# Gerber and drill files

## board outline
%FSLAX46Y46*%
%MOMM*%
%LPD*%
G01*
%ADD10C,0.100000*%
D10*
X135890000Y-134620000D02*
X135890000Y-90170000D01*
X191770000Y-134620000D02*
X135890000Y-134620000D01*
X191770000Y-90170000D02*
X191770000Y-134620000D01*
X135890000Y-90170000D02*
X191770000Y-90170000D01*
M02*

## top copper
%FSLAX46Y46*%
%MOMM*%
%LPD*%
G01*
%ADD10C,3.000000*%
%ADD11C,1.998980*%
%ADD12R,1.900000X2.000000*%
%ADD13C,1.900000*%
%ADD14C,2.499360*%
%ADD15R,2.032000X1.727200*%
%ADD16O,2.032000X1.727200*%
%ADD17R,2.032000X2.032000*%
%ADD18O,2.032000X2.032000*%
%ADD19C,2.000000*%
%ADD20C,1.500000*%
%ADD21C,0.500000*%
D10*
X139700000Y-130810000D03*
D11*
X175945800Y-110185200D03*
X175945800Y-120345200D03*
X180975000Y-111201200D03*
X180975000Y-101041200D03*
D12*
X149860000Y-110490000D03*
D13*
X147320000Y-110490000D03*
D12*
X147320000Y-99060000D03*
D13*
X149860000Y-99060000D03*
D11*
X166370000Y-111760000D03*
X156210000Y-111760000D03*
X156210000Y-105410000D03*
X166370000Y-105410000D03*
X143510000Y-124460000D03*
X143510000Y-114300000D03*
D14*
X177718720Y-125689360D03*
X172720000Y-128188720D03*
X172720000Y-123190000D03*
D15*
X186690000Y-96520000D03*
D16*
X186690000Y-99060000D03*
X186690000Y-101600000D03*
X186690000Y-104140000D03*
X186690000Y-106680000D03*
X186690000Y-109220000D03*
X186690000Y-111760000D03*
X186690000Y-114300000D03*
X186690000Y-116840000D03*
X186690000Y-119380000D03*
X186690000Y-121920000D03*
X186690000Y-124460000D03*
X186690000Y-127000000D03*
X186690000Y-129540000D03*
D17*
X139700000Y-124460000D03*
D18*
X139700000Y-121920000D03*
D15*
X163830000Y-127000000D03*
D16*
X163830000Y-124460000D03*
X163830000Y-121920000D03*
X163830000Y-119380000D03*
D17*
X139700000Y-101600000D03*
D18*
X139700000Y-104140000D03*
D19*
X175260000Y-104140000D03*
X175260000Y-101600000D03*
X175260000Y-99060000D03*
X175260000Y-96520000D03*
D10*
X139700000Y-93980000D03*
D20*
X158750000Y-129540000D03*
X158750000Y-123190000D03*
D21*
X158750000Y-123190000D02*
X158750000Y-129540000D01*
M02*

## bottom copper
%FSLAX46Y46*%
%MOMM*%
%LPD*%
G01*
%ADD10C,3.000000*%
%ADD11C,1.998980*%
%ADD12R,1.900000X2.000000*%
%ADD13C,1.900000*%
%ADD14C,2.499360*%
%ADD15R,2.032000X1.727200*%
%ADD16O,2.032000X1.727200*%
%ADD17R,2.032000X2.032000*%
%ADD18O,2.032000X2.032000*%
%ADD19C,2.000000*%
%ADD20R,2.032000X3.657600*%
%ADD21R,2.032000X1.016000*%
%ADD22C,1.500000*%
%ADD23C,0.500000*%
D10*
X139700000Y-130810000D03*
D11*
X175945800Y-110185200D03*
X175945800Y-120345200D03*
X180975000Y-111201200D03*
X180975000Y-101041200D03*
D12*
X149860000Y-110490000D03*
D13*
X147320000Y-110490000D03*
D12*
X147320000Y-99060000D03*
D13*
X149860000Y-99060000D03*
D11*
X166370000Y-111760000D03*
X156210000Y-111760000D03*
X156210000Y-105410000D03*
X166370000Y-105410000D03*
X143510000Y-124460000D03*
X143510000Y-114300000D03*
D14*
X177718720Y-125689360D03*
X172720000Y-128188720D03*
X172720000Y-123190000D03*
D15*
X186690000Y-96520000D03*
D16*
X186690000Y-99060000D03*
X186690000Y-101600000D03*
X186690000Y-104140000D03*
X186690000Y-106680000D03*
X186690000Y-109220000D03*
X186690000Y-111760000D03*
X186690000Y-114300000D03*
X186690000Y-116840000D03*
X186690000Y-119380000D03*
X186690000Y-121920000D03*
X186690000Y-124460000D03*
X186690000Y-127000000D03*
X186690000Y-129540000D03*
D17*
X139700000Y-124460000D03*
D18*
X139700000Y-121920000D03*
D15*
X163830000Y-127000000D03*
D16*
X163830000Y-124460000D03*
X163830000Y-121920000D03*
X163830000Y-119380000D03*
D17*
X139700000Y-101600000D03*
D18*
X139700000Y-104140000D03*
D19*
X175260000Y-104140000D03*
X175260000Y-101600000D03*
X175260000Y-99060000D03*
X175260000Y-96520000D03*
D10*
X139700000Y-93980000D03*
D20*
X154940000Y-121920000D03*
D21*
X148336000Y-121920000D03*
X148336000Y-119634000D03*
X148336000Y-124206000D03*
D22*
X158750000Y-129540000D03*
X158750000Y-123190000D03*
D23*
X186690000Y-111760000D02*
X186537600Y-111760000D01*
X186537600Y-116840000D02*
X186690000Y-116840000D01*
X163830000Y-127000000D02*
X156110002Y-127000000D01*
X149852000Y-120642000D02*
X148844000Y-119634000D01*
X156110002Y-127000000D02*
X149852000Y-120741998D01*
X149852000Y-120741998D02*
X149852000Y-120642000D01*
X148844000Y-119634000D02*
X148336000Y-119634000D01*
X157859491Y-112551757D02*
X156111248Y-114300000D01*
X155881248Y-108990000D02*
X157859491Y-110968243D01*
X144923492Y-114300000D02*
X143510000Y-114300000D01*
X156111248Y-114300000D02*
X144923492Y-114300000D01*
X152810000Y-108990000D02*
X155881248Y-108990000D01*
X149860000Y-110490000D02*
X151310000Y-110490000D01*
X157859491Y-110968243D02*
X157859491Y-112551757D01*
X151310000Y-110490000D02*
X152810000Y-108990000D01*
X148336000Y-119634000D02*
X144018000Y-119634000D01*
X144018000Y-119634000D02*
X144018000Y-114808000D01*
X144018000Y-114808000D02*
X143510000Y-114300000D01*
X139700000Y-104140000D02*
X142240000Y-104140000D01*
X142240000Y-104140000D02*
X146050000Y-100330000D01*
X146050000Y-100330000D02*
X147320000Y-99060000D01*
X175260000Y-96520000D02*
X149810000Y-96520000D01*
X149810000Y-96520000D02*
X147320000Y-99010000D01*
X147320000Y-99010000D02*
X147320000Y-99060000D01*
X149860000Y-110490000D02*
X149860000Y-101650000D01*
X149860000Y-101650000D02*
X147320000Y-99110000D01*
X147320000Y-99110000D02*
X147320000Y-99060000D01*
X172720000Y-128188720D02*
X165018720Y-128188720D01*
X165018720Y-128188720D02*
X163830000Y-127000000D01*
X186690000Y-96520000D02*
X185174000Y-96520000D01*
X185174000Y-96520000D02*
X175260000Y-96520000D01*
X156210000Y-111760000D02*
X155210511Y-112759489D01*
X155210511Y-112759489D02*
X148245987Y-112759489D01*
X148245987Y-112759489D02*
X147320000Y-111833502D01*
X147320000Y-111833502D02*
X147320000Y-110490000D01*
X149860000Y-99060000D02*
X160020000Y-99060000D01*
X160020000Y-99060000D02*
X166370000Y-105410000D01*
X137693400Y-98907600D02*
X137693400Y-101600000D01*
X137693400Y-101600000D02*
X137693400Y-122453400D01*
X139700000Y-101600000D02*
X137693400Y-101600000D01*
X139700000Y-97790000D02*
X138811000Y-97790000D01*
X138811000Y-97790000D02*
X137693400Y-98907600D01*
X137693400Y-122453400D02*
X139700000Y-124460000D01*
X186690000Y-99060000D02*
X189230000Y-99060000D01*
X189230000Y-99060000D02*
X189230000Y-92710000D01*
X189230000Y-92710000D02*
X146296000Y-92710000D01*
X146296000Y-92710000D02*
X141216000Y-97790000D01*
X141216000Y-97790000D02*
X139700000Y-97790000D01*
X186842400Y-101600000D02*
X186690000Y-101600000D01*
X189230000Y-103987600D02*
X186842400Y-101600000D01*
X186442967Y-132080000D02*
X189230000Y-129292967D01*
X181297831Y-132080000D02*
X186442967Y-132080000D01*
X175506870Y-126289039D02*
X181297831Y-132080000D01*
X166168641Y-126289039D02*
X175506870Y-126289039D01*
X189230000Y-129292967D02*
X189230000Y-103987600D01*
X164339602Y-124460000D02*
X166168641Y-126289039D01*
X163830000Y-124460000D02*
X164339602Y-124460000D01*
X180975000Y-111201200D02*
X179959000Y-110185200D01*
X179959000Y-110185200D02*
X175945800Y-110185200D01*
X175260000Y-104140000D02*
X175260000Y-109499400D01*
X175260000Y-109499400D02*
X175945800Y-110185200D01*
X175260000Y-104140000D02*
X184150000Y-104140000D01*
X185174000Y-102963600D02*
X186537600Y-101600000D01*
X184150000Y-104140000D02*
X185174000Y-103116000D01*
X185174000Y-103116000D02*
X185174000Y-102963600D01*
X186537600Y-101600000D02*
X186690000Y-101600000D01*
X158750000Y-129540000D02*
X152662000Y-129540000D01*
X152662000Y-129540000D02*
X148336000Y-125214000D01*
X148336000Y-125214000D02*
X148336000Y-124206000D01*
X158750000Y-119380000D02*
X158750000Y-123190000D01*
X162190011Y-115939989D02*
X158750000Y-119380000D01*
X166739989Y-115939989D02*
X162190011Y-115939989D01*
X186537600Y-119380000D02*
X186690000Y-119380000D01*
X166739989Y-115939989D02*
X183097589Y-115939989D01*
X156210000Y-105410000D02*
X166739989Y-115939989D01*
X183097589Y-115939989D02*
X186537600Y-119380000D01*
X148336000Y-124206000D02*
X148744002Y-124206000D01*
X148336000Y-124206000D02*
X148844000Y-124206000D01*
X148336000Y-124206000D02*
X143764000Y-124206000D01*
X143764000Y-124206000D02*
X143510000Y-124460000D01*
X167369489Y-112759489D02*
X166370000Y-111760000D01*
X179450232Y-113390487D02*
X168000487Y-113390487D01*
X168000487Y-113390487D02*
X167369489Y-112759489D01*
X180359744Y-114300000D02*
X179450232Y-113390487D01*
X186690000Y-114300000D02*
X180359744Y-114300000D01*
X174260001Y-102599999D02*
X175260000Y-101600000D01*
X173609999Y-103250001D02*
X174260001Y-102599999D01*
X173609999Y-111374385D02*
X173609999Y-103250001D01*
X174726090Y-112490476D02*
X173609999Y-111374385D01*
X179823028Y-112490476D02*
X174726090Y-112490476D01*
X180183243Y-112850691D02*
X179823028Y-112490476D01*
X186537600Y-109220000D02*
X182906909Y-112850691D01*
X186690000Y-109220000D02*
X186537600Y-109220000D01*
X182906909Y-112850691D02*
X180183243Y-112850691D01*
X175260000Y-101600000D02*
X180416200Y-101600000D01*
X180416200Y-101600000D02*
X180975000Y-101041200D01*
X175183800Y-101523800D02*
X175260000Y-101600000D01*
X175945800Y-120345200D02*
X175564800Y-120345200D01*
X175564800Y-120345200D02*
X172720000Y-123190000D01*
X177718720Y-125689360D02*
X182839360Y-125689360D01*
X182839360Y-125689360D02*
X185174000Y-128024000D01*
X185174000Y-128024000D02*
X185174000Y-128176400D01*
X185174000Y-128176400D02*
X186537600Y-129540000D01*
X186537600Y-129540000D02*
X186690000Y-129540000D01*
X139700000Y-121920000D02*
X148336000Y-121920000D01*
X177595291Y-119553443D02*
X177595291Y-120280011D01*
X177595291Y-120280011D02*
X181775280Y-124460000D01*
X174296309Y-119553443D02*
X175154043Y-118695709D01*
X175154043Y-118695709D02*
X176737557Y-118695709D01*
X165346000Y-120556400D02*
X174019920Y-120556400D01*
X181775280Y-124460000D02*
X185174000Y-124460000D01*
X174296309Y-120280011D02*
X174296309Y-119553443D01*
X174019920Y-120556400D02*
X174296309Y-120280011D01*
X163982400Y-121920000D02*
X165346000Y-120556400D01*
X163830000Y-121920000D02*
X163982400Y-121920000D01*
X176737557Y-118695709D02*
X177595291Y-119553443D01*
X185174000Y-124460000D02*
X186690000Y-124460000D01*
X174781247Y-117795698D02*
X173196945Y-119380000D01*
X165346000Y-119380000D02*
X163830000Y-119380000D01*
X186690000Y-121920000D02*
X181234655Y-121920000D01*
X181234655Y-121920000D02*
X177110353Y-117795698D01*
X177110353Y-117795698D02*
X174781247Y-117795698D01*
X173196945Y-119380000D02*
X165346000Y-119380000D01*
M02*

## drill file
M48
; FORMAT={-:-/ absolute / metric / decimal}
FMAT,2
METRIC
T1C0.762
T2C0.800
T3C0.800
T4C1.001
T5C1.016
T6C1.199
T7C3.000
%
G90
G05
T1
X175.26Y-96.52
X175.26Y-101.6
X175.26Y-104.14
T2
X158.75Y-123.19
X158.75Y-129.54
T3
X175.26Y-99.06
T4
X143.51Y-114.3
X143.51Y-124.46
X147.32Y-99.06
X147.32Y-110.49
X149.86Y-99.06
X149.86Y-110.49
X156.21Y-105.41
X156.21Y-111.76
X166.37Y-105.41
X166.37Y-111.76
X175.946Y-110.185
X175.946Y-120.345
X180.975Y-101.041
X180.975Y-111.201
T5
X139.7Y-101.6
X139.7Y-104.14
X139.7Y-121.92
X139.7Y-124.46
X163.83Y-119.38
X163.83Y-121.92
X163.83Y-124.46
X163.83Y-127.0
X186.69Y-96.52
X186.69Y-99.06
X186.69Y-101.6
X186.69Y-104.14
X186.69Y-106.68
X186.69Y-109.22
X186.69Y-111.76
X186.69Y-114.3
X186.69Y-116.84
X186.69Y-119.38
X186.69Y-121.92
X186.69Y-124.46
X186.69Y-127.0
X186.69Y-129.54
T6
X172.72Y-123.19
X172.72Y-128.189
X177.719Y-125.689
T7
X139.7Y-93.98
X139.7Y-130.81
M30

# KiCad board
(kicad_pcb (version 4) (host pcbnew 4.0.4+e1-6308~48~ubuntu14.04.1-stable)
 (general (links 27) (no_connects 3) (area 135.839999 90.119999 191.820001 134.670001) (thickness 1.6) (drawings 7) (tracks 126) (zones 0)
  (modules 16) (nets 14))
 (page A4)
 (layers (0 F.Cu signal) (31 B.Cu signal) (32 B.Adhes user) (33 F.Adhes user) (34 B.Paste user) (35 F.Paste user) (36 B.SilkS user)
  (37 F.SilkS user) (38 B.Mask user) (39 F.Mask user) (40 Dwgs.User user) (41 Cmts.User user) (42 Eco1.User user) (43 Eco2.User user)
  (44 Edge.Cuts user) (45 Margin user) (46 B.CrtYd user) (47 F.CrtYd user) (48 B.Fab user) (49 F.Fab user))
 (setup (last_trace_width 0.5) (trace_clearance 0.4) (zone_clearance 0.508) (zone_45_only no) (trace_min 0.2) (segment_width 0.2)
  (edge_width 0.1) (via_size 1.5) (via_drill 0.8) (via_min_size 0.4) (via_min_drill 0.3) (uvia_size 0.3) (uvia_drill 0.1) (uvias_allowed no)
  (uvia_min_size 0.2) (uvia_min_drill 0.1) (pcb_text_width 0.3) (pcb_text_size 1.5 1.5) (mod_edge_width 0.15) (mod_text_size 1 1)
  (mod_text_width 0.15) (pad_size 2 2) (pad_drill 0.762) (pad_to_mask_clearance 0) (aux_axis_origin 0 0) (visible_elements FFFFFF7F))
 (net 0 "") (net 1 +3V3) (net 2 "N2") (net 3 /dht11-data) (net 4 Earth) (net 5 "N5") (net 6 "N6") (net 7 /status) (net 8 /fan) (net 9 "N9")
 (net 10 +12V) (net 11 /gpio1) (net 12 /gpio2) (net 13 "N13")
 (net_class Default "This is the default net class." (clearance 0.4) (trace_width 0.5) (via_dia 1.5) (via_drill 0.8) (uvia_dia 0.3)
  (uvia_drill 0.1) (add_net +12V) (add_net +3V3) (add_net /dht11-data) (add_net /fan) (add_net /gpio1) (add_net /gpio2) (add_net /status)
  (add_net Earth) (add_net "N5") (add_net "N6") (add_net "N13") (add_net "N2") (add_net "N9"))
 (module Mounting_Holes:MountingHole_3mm (layer F.Cu) (at 139.7 130.81)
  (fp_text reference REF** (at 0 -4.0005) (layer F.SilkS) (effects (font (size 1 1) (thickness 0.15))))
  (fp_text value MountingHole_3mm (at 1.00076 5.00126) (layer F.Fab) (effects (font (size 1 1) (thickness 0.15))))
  (pad 1 thru_hole circle (at 0 0) (size 3 3) (drill 3) (layers)))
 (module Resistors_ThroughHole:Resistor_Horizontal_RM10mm (layer F.Cu) (at 175.9458 115.2652 270)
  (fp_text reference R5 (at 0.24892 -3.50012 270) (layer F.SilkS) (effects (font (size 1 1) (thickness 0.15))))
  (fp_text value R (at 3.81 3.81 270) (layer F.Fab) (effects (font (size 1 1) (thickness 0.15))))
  (pad 1 thru_hole circle (at -5.08 0 270) (size 1.99898 1.99898) (drill 1.00076) (layers *.Cu *.SilkS *.Mask) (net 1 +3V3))
  (pad 2 thru_hole circle (at 5.08 0 270) (size 1.99898 1.99898) (drill 1.00076) (layers *.Cu *.SilkS *.Mask) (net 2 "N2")))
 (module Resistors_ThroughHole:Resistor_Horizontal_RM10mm (layer F.Cu) (at 180.975 106.1212 90)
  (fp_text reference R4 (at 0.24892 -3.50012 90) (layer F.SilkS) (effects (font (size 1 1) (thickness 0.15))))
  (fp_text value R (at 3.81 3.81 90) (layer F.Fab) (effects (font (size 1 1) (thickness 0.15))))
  (pad 1 thru_hole circle (at -5.08 0 90) (size 1.99898 1.99898) (drill 1.00076) (layers *.Cu *.SilkS *.Mask) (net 1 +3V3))
  (pad 2 thru_hole circle (at 5.08 0 90) (size 1.99898 1.99898) (drill 1.00076) (layers *.Cu *.SilkS *.Mask) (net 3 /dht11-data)))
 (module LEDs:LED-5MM (layer F.Cu) (at 149.86 110.49 180)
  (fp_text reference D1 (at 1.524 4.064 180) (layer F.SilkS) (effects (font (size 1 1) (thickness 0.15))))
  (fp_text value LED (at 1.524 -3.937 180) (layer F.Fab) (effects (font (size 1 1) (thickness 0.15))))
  (pad 1 thru_hole rect (at 0 0 270) (size 2 1.9) (drill 1.00076) (layers *.Cu *.Mask F.SilkS) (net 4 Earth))
  (pad 2 thru_hole circle (at 2.54 0 180) (size 1.9 1.9) (drill 1.00076) (layers *.Cu *.Mask F.SilkS) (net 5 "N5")))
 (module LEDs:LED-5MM (layer F.Cu) (at 147.32 99.06)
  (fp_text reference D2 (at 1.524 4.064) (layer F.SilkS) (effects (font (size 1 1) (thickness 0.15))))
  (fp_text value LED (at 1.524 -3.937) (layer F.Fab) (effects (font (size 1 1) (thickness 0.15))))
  (pad 1 thru_hole rect (at 0 0 90) (size 2 1.9) (drill 1.00076) (layers *.Cu *.Mask F.SilkS) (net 4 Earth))
  (pad 2 thru_hole circle (at 2.54 0) (size 1.9 1.9) (drill 1.00076) (layers *.Cu *.Mask F.SilkS) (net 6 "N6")))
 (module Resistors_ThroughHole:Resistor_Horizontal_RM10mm (layer F.Cu) (at 161.29 111.76 180)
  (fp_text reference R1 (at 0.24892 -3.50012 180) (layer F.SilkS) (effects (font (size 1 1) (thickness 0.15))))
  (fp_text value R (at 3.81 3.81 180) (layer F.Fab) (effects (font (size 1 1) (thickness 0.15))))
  (pad 1 thru_hole circle (at -5.08 0 180) (size 1.99898 1.99898) (drill 1.00076) (layers *.Cu *.SilkS *.Mask) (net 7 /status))
  (pad 2 thru_hole circle (at 5.08 0 180) (size 1.99898 1.99898) (drill 1.00076) (layers *.Cu *.SilkS *.Mask) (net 5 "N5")))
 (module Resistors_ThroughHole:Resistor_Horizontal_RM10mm (layer F.Cu) (at 161.29 105.41)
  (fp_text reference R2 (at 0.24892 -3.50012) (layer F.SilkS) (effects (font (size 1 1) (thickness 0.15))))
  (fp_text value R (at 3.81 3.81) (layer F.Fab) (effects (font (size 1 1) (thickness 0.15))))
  (pad 1 thru_hole circle (at -5.08 0) (size 1.99898 1.99898) (drill 1.00076) (layers *.Cu *.SilkS *.Mask) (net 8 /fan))
  (pad 2 thru_hole circle (at 5.08 0) (size 1.99898 1.99898) (drill 1.00076) (layers *.Cu *.SilkS *.Mask) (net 6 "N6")))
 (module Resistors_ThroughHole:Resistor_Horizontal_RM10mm (layer F.Cu) (at 143.51 119.38 90)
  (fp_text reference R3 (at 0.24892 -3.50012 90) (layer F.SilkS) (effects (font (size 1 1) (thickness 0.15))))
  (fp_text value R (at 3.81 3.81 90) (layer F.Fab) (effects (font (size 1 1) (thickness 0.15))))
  (pad 1 thru_hole circle (at -5.08 0 90) (size 1.99898 1.99898) (drill 1.00076) (layers *.Cu *.SilkS *.Mask) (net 8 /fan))
  (pad 2 thru_hole circle (at 5.08 0 90) (size 1.99898 1.99898) (drill 1.00076) (layers *.Cu *.SilkS *.Mask) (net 4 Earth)))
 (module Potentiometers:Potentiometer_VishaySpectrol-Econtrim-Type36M (layer F.Cu) (at 172.72 123.19 270)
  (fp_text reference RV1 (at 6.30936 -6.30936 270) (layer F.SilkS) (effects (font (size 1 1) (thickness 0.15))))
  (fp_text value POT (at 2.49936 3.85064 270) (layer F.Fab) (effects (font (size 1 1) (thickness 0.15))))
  (pad 2 thru_hole circle (at 2.49936 -4.99872 270) (size 2.49936 2.49936) (drill 1.19888) (layers *.Cu *.Mask F.SilkS) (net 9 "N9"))
  (pad 3 thru_hole circle (at 4.99872 0 270) (size 2.49936 2.49936) (drill 1.19888) (layers *.Cu *.Mask F.SilkS) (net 4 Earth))
  (pad 1 thru_hole circle (at 0 0 270) (size 2.49936 2.49936) (drill 1.19888) (layers *.Cu *.Mask F.SilkS) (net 2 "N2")))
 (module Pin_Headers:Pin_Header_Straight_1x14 (layer F.Cu) (at 186.69 96.52)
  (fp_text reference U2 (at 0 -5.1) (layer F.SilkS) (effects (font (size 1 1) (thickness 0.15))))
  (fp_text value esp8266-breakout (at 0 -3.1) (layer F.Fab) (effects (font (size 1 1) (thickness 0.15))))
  (pad 1 thru_hole rect (at 0 0) (size 2.032 1.7272) (drill 1.016) (layers *.Cu *.Mask F.SilkS) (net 4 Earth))
  (pad 2 thru_hole oval (at 0 2.54) (size 2.032 1.7272) (drill 1.016) (layers *.Cu *.Mask F.SilkS) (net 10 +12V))
  (pad 3 thru_hole oval (at 0 5.08) (size 2.032 1.7272) (drill 1.016) (layers *.Cu *.Mask F.SilkS) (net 1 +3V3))
  (pad 4 thru_hole oval (at 0 7.62) (size 2.032 1.7272) (drill 1.016) (layers *.Cu *.Mask F.SilkS))
  (pad 5 thru_hole oval (at 0 10.16) (size 2.032 1.7272) (drill 1.016) (layers *.Cu *.Mask F.SilkS))
  (pad 6 thru_hole oval (at 0 12.7) (size 2.032 1.7272) (drill 1.016) (layers *.Cu *.Mask F.SilkS) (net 3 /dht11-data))
  (pad 7 thru_hole oval (at 0 15.24) (size 2.032 1.7272) (drill 1.016) (layers *.Cu *.Mask F.SilkS))
  (pad 8 thru_hole oval (at 0 17.78) (size 2.032 1.7272) (drill 1.016) (layers *.Cu *.Mask F.SilkS) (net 7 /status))
  (pad 9 thru_hole oval (at 0 20.32) (size 2.032 1.7272) (drill 1.016) (layers *.Cu *.Mask F.SilkS))
  (pad 10 thru_hole oval (at 0 22.86) (size 2.032 1.7272) (drill 1.016) (layers *.Cu *.Mask F.SilkS) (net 8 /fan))
  (pad 11 thru_hole oval (at 0 25.4) (size 2.032 1.7272) (drill 1.016) (layers *.Cu *.Mask F.SilkS) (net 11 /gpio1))
  (pad 12 thru_hole oval (at 0 27.94) (size 2.032 1.7272) (drill 1.016) (layers *.Cu *.Mask F.SilkS) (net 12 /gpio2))
  (pad 13 thru_hole oval (at 0 30.48) (size 2.032 1.7272) (drill 1.016) (layers *.Cu *.Mask F.SilkS))
  (pad 14 thru_hole oval (at 0 33.02) (size 2.032 1.7272) (drill 1.016) (layers *.Cu *.Mask F.SilkS) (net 9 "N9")))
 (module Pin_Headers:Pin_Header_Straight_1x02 (layer F.Cu) (at 139.7 124.46 180)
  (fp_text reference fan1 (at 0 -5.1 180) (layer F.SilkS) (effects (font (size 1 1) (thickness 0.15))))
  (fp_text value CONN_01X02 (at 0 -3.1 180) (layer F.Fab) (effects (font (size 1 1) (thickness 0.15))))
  (pad 1 thru_hole rect (at 0 0 180) (size 2.032 2.032) (drill 1.016) (layers *.Cu *.Mask F.SilkS) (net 10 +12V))
  (pad 2 thru_hole oval (at 0 2.54 180) (size 2.032 2.032) (drill 1.016) (layers *.Cu *.Mask F.SilkS) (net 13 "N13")))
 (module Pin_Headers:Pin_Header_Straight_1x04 (layer F.Cu) (at 163.83 127 180)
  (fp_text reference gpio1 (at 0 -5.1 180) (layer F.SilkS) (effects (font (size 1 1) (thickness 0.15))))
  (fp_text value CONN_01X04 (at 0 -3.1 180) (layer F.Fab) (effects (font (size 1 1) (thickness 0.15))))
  (pad 1 thru_hole rect (at 0 0 180) (size 2.032 1.7272) (drill 1.016) (layers *.Cu *.Mask F.SilkS) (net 4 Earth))
  (pad 2 thru_hole oval (at 0 2.54 180) (size 2.032 1.7272) (drill 1.016) (layers *.Cu *.Mask F.SilkS) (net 1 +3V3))
  (pad 3 thru_hole oval (at 0 5.08 180) (size 2.032 1.7272) (drill 1.016) (layers *.Cu *.Mask F.SilkS) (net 12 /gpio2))
  (pad 4 thru_hole oval (at 0 7.62 180) (size 2.032 1.7272) (drill 1.016) (layers *.Cu *.Mask F.SilkS) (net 11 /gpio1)))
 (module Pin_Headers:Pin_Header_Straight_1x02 (layer F.Cu) (at 139.7 101.6)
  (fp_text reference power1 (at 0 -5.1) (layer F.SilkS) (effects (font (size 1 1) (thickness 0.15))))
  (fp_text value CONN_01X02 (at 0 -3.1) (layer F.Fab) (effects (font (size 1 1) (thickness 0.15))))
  (pad 1 thru_hole rect (at 0 0) (size 2.032 2.032) (drill 1.016) (layers *.Cu *.Mask F.SilkS) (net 10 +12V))
  (pad 2 thru_hole oval (at 0 2.54) (size 2.032 2.032) (drill 1.016) (layers *.Cu *.Mask F.SilkS) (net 4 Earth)))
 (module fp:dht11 (layer F.Cu) (at 175.26 93.98 180)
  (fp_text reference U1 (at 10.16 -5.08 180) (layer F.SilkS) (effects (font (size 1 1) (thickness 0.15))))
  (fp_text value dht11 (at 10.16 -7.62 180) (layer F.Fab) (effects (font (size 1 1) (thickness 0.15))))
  (pad 1 thru_hole circle (at 0 -10.16 180) (size 2 2) (drill 0.762) (layers *.Cu *.Mask F.SilkS) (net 1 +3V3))
  (pad 2 thru_hole circle (at 0 -7.62 180) (size 2 2) (drill 0.762) (layers *.Cu *.Mask F.SilkS) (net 3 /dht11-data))
  (pad 3 thru_hole circle (at 0 -5.08 180) (size 2 2) (drill 0.8) (layers *.Cu *.Mask F.SilkS))
  (pad 4 thru_hole circle (at 0 -2.54 180) (size 2 2) (drill 0.762) (layers *.Cu *.Mask F.SilkS) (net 4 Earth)))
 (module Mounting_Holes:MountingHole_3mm (layer F.Cu) (at 139.7 93.98)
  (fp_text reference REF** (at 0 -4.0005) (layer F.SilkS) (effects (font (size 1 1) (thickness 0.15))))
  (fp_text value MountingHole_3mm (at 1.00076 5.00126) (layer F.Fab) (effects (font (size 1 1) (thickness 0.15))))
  (pad 1 thru_hole circle (at 0 0) (size 3 3) (drill 3) (layers)))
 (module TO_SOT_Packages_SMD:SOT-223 (layer B.Cu) (at 151.638 121.92 90)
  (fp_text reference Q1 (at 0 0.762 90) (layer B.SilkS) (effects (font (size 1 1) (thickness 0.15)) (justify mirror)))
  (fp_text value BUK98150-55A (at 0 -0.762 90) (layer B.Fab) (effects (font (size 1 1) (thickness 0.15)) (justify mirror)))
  (pad 4 smd rect (at 0 3.302 90) (size 3.6576 2.032) (layers B.Cu B.Paste B.Mask))
  (pad 2 smd rect (at 0 -3.302 90) (size 1.016 2.032) (layers B.Cu B.Paste B.Mask) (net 13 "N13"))
  (pad 3 smd rect (at 2.286 -3.302 90) (size 1.016 2.032) (layers B.Cu B.Paste B.Mask) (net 4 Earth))
  (pad 1 smd rect (at -2.286 -3.302 90) (size 1.016 2.032) (layers B.Cu B.Paste B.Mask) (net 8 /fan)))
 (gr_line (start 135.89 134.62) (end 135.89 90.17) (layer Edge.Cuts) (width 0.1))
 (gr_line (start 191.77 134.62) (end 135.89 134.62) (layer Edge.Cuts) (width 0.1))
 (gr_line (start 191.77 90.17) (end 191.77 134.62) (layer Edge.Cuts) (width 0.1))
 (gr_line (start 135.89 90.17) (end 191.77 90.17) (layer Edge.Cuts) (width 0.1))
 (segment (start 186.69 111.76) (end 186.5376 111.76) (width 0.5) (layer B.Cu) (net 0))
 (segment (start 186.5376 116.84) (end 186.69 116.84) (width 0.5) (layer B.Cu) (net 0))
 (segment (start 163.83 127) (end 156.110002 127) (width 0.5) (layer B.Cu) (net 4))
 (segment (start 149.852 120.642) (end 148.844 119.634) (width 0.5) (layer B.Cu) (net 4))
 (segment (start 156.110002 127) (end 149.852 120.741998) (width 0.5) (layer B.Cu) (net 4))
 (segment (start 149.852 120.741998) (end 149.852 120.642) (width 0.5) (layer B.Cu) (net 4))
 (segment (start 148.844 119.634) (end 148.336 119.634) (width 0.5) (layer B.Cu) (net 4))
 (segment (start 157.859491 112.551757) (end 156.111248 114.3) (width 0.5) (layer B.Cu) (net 4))
 (segment (start 155.881248 108.99) (end 157.859491 110.968243) (width 0.5) (layer B.Cu) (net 4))
 (segment (start 144.923492 114.3) (end 143.51 114.3) (width 0.5) (layer B.Cu) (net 4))
 (segment (start 156.111248 114.3) (end 144.923492 114.3) (width 0.5) (layer B.Cu) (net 4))
 (segment (start 152.81 108.99) (end 155.881248 108.99) (width 0.5) (layer B.Cu) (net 4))
 (segment (start 149.86 110.49) (end 151.31 110.49) (width 0.5) (layer B.Cu) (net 4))
 (segment (start 157.859491 110.968243) (end 157.859491 112.551757) (width 0.5) (layer B.Cu) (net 4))
 (segment (start 151.31 110.49) (end 152.81 108.99) (width 0.5) (layer B.Cu) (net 4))
 (segment (start 148.336 119.634) (end 144.018 119.634) (width 0.5) (layer B.Cu) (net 4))
 (segment (start 144.018 119.634) (end 144.018 114.808) (width 0.5) (layer B.Cu) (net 4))
 (segment (start 144.018 114.808) (end 143.51 114.3) (width 0.5) (layer B.Cu) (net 4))
 (segment (start 139.7 104.14) (end 142.24 104.14) (width 0.5) (layer B.Cu) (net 4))
 (segment (start 142.24 104.14) (end 146.05 100.33) (width 0.5) (layer B.Cu) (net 4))
 (segment (start 146.05 100.33) (end 147.32 99.06) (width 0.5) (layer B.Cu) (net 4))
 (segment (start 175.26 96.52) (end 149.81 96.52) (width 0.5) (layer B.Cu) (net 4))
 (segment (start 149.81 96.52) (end 147.32 99.01) (width 0.5) (layer B.Cu) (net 4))
 (segment (start 147.32 99.01) (end 147.32 99.06) (width 0.5) (layer B.Cu) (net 4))
 (segment (start 149.86 110.49) (end 149.86 101.65) (width 0.5) (layer B.Cu) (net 4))
 (segment (start 149.86 101.65) (end 147.32 99.11) (width 0.5) (layer B.Cu) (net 4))
 (segment (start 147.32 99.11) (end 147.32 99.06) (width 0.5) (layer B.Cu) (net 4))
 (segment (start 172.72 128.18872) (end 165.01872 128.18872) (width 0.5) (layer B.Cu) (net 4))
 (segment (start 165.01872 128.18872) (end 163.83 127) (width 0.5) (layer B.Cu) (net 4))
 (segment (start 186.69 96.52) (end 185.174 96.52) (width 0.5) (layer B.Cu) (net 4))
 (segment (start 185.174 96.52) (end 175.26 96.52) (width 0.5) (layer B.Cu) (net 4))
 (segment (start 156.21 111.76) (end 155.210511 112.759489) (width 0.5) (layer B.Cu) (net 5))
 (segment (start 155.210511 112.759489) (end 148.245987 112.759489) (width 0.5) (layer B.Cu) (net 5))
 (segment (start 148.245987 112.759489) (end 147.32 111.833502) (width 0.5) (layer B.Cu) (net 5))
 (segment (start 147.32 111.833502) (end 147.32 110.49) (width 0.5) (layer B.Cu) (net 5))
 (segment (start 149.86 99.06) (end 160.02 99.06) (width 0.5) (layer B.Cu) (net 6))
 (segment (start 160.02 99.06) (end 166.37 105.41) (width 0.5) (layer B.Cu) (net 6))
 (segment (start 137.6934 98.9076) (end 137.6934 101.6) (width 0.5) (layer B.Cu) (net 10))
 (segment (start 137.6934 101.6) (end 137.6934 122.4534) (width 0.5) (layer B.Cu) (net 10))
 (segment (start 139.7 101.6) (end 137.6934 101.6) (width 0.5) (layer B.Cu) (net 10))
 (segment (start 139.7 97.79) (end 138.811 97.79) (width 0.5) (layer B.Cu) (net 10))
 (segment (start 138.811 97.79) (end 137.6934 98.9076) (width 0.5) (layer B.Cu) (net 10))
 (segment (start 137.6934 122.4534) (end 139.7 124.46) (width 0.5) (layer B.Cu) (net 10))
 (segment (start 186.69 99.06) (end 189.23 99.06) (width 0.5) (layer B.Cu) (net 10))
 (segment (start 189.23 99.06) (end 189.23 92.71) (width 0.5) (layer B.Cu) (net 10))
 (segment (start 189.23 92.71) (end 146.296 92.71) (width 0.5) (layer B.Cu) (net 10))
 (segment (start 146.296 92.71) (end 141.216 97.79) (width 0.5) (layer B.Cu) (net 10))
 (segment (start 141.216 97.79) (end 139.7 97.79) (width 0.5) (layer B.Cu) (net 10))
 (segment (start 186.8424 101.6) (end 186.69 101.6) (width 0.5) (layer B.Cu) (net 1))
 (segment (start 189.23 103.9876) (end 186.8424 101.6) (width 0.5) (layer B.Cu) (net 1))
 (segment (start 186.442967 132.08) (end 189.23 129.292967) (width 0.5) (layer B.Cu) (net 1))
 (segment (start 181.297831 132.08) (end 186.442967 132.08) (width 0.5) (layer B.Cu) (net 1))
 (segment (start 175.50687 126.289039) (end 181.297831 132.08) (width 0.5) (layer B.Cu) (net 1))
 (segment (start 166.168641 126.289039) (end 175.50687 126.289039) (width 0.5) (layer B.Cu) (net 1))
 (segment (start 189.23 129.292967) (end 189.23 103.9876) (width 0.5) (layer B.Cu) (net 1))
 (segment (start 164.339602 124.46) (end 166.168641 126.289039) (width 0.5) (layer B.Cu) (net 1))
 (segment (start 163.83 124.46) (end 164.339602 124.46) (width 0.5) (layer B.Cu) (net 1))
 (segment (start 180.975 111.2012) (end 179.959 110.1852) (width 0.5) (layer B.Cu) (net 1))
 (segment (start 179.959 110.1852) (end 175.9458 110.1852) (width 0.5) (layer B.Cu) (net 1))
 (segment (start 175.26 104.14) (end 175.26 109.4994) (width 0.5) (layer B.Cu) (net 1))
 (segment (start 175.26 109.4994) (end 175.9458 110.1852) (width 0.5) (layer B.Cu) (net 1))
 (segment (start 175.26 104.14) (end 184.15 104.14) (width 0.5) (layer B.Cu) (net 1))
 (segment (start 185.174 102.9636) (end 186.5376 101.6) (width 0.5) (layer B.Cu) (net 1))
 (segment (start 184.15 104.14) (end 185.174 103.116) (width 0.5) (layer B.Cu) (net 1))
 (segment (start 185.174 103.116) (end 185.174 102.9636) (width 0.5) (layer B.Cu) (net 1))
 (segment (start 186.5376 101.6) (end 186.69 101.6) (width 0.5) (layer B.Cu) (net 1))
 (segment (start 158.75 129.54) (end 152.662 129.54) (width 0.5) (layer B.Cu) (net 8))
 (segment (start 152.662 129.54) (end 148.336 125.214) (width 0.5) (layer B.Cu) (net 8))
 (segment (start 148.336 125.214) (end 148.336 124.206) (width 0.5) (layer B.Cu) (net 8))
 (segment (start 158.75 123.19) (end 158.75 129.54) (width 0.5) (layer F.Cu) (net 8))
 (via (at 158.75 129.54) (size 1.5) (drill 0.8) (layers F.Cu B.Cu) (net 8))
 (segment (start 158.75 119.38) (end 158.75 123.19) (width 0.5) (layer B.Cu) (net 8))
 (via (at 158.75 123.19) (size 1.5) (drill 0.8) (layers F.Cu B.Cu) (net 8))
 (segment (start 162.190011 115.939989) (end 158.75 119.38) (width 0.5) (layer B.Cu) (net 8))
 (segment (start 166.739989 115.939989) (end 162.190011 115.939989) (width 0.5) (layer B.Cu) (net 8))
 (segment (start 186.5376 119.38) (end 186.69 119.38) (width 0.5) (layer B.Cu) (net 8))
 (segment (start 166.739989 115.939989) (end 183.097589 115.939989) (width 0.5) (layer B.Cu) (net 8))
 (segment (start 156.21 105.41) (end 166.739989 115.939989) (width 0.5) (layer B.Cu) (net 8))
 (segment (start 183.097589 115.939989) (end 186.5376 119.38) (width 0.5) (layer B.Cu) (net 8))
 (segment (start 148.336 124.206) (end 148.744002 124.206) (width 0.5) (layer B.Cu) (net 8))
 (segment (start 148.336 124.206) (end 148.844 124.206) (width 0.5) (layer B.Cu) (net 8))
 (segment (start 148.336 124.206) (end 143.764 124.206) (width 0.5) (layer B.Cu) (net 8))
 (segment (start 143.764 124.206) (end 143.51 124.46) (width 0.5) (layer B.Cu) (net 8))
 (segment (start 167.369489 112.759489) (end 166.37 111.76) (width 0.5) (layer B.Cu) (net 7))
 (segment (start 179.450232 113.390487) (end 168.000487 113.390487) (width 0.5) (layer B.Cu) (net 7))
 (segment (start 168.000487 113.390487) (end 167.369489 112.759489) (width 0.5) (layer B.Cu) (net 7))
 (segment (start 180.359744 114.3) (end 179.450232 113.390487) (width 0.5) (layer B.Cu) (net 7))
 (segment (start 186.69 114.3) (end 180.359744 114.3) (width 0.5) (layer B.Cu) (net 7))
 (segment (start 174.260001 102.599999) (end 175.26 101.6) (width 0.5) (layer B.Cu) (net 3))
 (segment (start 173.609999 103.250001) (end 174.260001 102.599999) (width 0.5) (layer B.Cu) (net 3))
 (segment (start 173.609999 111.374385) (end 173.609999 103.250001) (width 0.5) (layer B.Cu) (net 3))
 (segment (start 174.72609 112.490476) (end 173.609999 111.374385) (width 0.5) (layer B.Cu) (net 3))
 (segment (start 179.823028 112.490476) (end 174.72609 112.490476) (width 0.5) (layer B.Cu) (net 3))
 (segment (start 180.183243 112.850691) (end 179.823028 112.490476) (width 0.5) (layer B.Cu) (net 3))
 (segment (start 186.5376 109.22) (end 182.906909 112.850691) (width 0.5) (layer B.Cu) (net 3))
 (segment (start 186.69 109.22) (end 186.5376 109.22) (width 0.5) (layer B.Cu) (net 3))
 (segment (start 182.906909 112.850691) (end 180.183243 112.850691) (width 0.5) (layer B.Cu) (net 3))
 (segment (start 175.26 101.6) (end 180.4162 101.6) (width 0.5) (layer B.Cu) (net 3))
 (segment (start 180.4162 101.6) (end 180.975 101.0412) (width 0.5) (layer B.Cu) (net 3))
 (segment (start 175.1838 101.5238) (end 175.26 101.6) (width 0.5) (layer B.Cu) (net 3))
 (segment (start 175.9458 120.3452) (end 175.5648 120.3452) (width 0.5) (layer B.Cu) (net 2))
 (segment (start 175.5648 120.3452) (end 172.72 123.19) (width 0.5) (layer B.Cu) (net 2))
 (segment (start 177.71872 125.68936) (end 182.83936 125.68936) (width 0.5) (layer B.Cu) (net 9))
 (segment (start 182.83936 125.68936) (end 185.174 128.024) (width 0.5) (layer B.Cu) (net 9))
 (segment (start 185.174 128.024) (end 185.174 128.1764) (width 0.5) (layer B.Cu) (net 9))
 (segment (start 185.174 128.1764) (end 186.5376 129.54) (width 0.5) (layer B.Cu) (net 9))
 (segment (start 186.5376 129.54) (end 186.69 129.54) (width 0.5) (layer B.Cu) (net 9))
 (segment (start 139.7 121.92) (end 148.336 121.92) (width 0.5) (layer B.Cu) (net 13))
 (segment (start 177.595291 119.553443) (end 177.595291 120.280011) (width 0.5) (layer B.Cu) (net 12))
 (segment (start 177.595291 120.280011) (end 181.77528 124.46) (width 0.5) (layer B.Cu) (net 12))
 (segment (start 174.296309 119.553443) (end 175.154043 118.695709) (width 0.5) (layer B.Cu) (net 12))
 (segment (start 175.154043 118.695709) (end 176.737557 118.695709) (width 0.5) (layer B.Cu) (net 12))
 (segment (start 165.346 120.5564) (end 174.01992 120.5564) (width 0.5) (layer B.Cu) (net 12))
 (segment (start 181.77528 124.46) (end 185.174 124.46) (width 0.5) (layer B.Cu) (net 12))
 (segment (start 174.296309 120.280011) (end 174.296309 119.553443) (width 0.5) (layer B.Cu) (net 12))
 (segment (start 174.01992 120.5564) (end 174.296309 120.280011) (width 0.5) (layer B.Cu) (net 12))
 (segment (start 163.9824 121.92) (end 165.346 120.5564) (width 0.5) (layer B.Cu) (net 12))
 (segment (start 163.83 121.92) (end 163.9824 121.92) (width 0.5) (layer B.Cu) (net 12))
 (segment (start 176.737557 118.695709) (end 177.595291 119.553443) (width 0.5) (layer B.Cu) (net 12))
 (segment (start 185.174 124.46) (end 186.69 124.46) (width 0.5) (layer B.Cu) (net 12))
 (segment (start 174.781247 117.795698) (end 173.196945 119.38) (width 0.5) (layer B.Cu) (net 11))
 (segment (start 165.346 119.38) (end 163.83 119.38) (width 0.5) (layer B.Cu) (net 11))
 (segment (start 186.69 121.92) (end 181.234655 121.92) (width 0.5) (layer B.Cu) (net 11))
 (segment (start 181.234655 121.92) (end 177.110353 117.795698) (width 0.5) (layer B.Cu) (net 11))
 (segment (start 177.110353 117.795698) (end 174.781247 117.795698) (width 0.5) (layer B.Cu) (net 11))
 (segment (start 173.196945 119.38) (end 165.346 119.38) (width 0.5) (layer B.Cu) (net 11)))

